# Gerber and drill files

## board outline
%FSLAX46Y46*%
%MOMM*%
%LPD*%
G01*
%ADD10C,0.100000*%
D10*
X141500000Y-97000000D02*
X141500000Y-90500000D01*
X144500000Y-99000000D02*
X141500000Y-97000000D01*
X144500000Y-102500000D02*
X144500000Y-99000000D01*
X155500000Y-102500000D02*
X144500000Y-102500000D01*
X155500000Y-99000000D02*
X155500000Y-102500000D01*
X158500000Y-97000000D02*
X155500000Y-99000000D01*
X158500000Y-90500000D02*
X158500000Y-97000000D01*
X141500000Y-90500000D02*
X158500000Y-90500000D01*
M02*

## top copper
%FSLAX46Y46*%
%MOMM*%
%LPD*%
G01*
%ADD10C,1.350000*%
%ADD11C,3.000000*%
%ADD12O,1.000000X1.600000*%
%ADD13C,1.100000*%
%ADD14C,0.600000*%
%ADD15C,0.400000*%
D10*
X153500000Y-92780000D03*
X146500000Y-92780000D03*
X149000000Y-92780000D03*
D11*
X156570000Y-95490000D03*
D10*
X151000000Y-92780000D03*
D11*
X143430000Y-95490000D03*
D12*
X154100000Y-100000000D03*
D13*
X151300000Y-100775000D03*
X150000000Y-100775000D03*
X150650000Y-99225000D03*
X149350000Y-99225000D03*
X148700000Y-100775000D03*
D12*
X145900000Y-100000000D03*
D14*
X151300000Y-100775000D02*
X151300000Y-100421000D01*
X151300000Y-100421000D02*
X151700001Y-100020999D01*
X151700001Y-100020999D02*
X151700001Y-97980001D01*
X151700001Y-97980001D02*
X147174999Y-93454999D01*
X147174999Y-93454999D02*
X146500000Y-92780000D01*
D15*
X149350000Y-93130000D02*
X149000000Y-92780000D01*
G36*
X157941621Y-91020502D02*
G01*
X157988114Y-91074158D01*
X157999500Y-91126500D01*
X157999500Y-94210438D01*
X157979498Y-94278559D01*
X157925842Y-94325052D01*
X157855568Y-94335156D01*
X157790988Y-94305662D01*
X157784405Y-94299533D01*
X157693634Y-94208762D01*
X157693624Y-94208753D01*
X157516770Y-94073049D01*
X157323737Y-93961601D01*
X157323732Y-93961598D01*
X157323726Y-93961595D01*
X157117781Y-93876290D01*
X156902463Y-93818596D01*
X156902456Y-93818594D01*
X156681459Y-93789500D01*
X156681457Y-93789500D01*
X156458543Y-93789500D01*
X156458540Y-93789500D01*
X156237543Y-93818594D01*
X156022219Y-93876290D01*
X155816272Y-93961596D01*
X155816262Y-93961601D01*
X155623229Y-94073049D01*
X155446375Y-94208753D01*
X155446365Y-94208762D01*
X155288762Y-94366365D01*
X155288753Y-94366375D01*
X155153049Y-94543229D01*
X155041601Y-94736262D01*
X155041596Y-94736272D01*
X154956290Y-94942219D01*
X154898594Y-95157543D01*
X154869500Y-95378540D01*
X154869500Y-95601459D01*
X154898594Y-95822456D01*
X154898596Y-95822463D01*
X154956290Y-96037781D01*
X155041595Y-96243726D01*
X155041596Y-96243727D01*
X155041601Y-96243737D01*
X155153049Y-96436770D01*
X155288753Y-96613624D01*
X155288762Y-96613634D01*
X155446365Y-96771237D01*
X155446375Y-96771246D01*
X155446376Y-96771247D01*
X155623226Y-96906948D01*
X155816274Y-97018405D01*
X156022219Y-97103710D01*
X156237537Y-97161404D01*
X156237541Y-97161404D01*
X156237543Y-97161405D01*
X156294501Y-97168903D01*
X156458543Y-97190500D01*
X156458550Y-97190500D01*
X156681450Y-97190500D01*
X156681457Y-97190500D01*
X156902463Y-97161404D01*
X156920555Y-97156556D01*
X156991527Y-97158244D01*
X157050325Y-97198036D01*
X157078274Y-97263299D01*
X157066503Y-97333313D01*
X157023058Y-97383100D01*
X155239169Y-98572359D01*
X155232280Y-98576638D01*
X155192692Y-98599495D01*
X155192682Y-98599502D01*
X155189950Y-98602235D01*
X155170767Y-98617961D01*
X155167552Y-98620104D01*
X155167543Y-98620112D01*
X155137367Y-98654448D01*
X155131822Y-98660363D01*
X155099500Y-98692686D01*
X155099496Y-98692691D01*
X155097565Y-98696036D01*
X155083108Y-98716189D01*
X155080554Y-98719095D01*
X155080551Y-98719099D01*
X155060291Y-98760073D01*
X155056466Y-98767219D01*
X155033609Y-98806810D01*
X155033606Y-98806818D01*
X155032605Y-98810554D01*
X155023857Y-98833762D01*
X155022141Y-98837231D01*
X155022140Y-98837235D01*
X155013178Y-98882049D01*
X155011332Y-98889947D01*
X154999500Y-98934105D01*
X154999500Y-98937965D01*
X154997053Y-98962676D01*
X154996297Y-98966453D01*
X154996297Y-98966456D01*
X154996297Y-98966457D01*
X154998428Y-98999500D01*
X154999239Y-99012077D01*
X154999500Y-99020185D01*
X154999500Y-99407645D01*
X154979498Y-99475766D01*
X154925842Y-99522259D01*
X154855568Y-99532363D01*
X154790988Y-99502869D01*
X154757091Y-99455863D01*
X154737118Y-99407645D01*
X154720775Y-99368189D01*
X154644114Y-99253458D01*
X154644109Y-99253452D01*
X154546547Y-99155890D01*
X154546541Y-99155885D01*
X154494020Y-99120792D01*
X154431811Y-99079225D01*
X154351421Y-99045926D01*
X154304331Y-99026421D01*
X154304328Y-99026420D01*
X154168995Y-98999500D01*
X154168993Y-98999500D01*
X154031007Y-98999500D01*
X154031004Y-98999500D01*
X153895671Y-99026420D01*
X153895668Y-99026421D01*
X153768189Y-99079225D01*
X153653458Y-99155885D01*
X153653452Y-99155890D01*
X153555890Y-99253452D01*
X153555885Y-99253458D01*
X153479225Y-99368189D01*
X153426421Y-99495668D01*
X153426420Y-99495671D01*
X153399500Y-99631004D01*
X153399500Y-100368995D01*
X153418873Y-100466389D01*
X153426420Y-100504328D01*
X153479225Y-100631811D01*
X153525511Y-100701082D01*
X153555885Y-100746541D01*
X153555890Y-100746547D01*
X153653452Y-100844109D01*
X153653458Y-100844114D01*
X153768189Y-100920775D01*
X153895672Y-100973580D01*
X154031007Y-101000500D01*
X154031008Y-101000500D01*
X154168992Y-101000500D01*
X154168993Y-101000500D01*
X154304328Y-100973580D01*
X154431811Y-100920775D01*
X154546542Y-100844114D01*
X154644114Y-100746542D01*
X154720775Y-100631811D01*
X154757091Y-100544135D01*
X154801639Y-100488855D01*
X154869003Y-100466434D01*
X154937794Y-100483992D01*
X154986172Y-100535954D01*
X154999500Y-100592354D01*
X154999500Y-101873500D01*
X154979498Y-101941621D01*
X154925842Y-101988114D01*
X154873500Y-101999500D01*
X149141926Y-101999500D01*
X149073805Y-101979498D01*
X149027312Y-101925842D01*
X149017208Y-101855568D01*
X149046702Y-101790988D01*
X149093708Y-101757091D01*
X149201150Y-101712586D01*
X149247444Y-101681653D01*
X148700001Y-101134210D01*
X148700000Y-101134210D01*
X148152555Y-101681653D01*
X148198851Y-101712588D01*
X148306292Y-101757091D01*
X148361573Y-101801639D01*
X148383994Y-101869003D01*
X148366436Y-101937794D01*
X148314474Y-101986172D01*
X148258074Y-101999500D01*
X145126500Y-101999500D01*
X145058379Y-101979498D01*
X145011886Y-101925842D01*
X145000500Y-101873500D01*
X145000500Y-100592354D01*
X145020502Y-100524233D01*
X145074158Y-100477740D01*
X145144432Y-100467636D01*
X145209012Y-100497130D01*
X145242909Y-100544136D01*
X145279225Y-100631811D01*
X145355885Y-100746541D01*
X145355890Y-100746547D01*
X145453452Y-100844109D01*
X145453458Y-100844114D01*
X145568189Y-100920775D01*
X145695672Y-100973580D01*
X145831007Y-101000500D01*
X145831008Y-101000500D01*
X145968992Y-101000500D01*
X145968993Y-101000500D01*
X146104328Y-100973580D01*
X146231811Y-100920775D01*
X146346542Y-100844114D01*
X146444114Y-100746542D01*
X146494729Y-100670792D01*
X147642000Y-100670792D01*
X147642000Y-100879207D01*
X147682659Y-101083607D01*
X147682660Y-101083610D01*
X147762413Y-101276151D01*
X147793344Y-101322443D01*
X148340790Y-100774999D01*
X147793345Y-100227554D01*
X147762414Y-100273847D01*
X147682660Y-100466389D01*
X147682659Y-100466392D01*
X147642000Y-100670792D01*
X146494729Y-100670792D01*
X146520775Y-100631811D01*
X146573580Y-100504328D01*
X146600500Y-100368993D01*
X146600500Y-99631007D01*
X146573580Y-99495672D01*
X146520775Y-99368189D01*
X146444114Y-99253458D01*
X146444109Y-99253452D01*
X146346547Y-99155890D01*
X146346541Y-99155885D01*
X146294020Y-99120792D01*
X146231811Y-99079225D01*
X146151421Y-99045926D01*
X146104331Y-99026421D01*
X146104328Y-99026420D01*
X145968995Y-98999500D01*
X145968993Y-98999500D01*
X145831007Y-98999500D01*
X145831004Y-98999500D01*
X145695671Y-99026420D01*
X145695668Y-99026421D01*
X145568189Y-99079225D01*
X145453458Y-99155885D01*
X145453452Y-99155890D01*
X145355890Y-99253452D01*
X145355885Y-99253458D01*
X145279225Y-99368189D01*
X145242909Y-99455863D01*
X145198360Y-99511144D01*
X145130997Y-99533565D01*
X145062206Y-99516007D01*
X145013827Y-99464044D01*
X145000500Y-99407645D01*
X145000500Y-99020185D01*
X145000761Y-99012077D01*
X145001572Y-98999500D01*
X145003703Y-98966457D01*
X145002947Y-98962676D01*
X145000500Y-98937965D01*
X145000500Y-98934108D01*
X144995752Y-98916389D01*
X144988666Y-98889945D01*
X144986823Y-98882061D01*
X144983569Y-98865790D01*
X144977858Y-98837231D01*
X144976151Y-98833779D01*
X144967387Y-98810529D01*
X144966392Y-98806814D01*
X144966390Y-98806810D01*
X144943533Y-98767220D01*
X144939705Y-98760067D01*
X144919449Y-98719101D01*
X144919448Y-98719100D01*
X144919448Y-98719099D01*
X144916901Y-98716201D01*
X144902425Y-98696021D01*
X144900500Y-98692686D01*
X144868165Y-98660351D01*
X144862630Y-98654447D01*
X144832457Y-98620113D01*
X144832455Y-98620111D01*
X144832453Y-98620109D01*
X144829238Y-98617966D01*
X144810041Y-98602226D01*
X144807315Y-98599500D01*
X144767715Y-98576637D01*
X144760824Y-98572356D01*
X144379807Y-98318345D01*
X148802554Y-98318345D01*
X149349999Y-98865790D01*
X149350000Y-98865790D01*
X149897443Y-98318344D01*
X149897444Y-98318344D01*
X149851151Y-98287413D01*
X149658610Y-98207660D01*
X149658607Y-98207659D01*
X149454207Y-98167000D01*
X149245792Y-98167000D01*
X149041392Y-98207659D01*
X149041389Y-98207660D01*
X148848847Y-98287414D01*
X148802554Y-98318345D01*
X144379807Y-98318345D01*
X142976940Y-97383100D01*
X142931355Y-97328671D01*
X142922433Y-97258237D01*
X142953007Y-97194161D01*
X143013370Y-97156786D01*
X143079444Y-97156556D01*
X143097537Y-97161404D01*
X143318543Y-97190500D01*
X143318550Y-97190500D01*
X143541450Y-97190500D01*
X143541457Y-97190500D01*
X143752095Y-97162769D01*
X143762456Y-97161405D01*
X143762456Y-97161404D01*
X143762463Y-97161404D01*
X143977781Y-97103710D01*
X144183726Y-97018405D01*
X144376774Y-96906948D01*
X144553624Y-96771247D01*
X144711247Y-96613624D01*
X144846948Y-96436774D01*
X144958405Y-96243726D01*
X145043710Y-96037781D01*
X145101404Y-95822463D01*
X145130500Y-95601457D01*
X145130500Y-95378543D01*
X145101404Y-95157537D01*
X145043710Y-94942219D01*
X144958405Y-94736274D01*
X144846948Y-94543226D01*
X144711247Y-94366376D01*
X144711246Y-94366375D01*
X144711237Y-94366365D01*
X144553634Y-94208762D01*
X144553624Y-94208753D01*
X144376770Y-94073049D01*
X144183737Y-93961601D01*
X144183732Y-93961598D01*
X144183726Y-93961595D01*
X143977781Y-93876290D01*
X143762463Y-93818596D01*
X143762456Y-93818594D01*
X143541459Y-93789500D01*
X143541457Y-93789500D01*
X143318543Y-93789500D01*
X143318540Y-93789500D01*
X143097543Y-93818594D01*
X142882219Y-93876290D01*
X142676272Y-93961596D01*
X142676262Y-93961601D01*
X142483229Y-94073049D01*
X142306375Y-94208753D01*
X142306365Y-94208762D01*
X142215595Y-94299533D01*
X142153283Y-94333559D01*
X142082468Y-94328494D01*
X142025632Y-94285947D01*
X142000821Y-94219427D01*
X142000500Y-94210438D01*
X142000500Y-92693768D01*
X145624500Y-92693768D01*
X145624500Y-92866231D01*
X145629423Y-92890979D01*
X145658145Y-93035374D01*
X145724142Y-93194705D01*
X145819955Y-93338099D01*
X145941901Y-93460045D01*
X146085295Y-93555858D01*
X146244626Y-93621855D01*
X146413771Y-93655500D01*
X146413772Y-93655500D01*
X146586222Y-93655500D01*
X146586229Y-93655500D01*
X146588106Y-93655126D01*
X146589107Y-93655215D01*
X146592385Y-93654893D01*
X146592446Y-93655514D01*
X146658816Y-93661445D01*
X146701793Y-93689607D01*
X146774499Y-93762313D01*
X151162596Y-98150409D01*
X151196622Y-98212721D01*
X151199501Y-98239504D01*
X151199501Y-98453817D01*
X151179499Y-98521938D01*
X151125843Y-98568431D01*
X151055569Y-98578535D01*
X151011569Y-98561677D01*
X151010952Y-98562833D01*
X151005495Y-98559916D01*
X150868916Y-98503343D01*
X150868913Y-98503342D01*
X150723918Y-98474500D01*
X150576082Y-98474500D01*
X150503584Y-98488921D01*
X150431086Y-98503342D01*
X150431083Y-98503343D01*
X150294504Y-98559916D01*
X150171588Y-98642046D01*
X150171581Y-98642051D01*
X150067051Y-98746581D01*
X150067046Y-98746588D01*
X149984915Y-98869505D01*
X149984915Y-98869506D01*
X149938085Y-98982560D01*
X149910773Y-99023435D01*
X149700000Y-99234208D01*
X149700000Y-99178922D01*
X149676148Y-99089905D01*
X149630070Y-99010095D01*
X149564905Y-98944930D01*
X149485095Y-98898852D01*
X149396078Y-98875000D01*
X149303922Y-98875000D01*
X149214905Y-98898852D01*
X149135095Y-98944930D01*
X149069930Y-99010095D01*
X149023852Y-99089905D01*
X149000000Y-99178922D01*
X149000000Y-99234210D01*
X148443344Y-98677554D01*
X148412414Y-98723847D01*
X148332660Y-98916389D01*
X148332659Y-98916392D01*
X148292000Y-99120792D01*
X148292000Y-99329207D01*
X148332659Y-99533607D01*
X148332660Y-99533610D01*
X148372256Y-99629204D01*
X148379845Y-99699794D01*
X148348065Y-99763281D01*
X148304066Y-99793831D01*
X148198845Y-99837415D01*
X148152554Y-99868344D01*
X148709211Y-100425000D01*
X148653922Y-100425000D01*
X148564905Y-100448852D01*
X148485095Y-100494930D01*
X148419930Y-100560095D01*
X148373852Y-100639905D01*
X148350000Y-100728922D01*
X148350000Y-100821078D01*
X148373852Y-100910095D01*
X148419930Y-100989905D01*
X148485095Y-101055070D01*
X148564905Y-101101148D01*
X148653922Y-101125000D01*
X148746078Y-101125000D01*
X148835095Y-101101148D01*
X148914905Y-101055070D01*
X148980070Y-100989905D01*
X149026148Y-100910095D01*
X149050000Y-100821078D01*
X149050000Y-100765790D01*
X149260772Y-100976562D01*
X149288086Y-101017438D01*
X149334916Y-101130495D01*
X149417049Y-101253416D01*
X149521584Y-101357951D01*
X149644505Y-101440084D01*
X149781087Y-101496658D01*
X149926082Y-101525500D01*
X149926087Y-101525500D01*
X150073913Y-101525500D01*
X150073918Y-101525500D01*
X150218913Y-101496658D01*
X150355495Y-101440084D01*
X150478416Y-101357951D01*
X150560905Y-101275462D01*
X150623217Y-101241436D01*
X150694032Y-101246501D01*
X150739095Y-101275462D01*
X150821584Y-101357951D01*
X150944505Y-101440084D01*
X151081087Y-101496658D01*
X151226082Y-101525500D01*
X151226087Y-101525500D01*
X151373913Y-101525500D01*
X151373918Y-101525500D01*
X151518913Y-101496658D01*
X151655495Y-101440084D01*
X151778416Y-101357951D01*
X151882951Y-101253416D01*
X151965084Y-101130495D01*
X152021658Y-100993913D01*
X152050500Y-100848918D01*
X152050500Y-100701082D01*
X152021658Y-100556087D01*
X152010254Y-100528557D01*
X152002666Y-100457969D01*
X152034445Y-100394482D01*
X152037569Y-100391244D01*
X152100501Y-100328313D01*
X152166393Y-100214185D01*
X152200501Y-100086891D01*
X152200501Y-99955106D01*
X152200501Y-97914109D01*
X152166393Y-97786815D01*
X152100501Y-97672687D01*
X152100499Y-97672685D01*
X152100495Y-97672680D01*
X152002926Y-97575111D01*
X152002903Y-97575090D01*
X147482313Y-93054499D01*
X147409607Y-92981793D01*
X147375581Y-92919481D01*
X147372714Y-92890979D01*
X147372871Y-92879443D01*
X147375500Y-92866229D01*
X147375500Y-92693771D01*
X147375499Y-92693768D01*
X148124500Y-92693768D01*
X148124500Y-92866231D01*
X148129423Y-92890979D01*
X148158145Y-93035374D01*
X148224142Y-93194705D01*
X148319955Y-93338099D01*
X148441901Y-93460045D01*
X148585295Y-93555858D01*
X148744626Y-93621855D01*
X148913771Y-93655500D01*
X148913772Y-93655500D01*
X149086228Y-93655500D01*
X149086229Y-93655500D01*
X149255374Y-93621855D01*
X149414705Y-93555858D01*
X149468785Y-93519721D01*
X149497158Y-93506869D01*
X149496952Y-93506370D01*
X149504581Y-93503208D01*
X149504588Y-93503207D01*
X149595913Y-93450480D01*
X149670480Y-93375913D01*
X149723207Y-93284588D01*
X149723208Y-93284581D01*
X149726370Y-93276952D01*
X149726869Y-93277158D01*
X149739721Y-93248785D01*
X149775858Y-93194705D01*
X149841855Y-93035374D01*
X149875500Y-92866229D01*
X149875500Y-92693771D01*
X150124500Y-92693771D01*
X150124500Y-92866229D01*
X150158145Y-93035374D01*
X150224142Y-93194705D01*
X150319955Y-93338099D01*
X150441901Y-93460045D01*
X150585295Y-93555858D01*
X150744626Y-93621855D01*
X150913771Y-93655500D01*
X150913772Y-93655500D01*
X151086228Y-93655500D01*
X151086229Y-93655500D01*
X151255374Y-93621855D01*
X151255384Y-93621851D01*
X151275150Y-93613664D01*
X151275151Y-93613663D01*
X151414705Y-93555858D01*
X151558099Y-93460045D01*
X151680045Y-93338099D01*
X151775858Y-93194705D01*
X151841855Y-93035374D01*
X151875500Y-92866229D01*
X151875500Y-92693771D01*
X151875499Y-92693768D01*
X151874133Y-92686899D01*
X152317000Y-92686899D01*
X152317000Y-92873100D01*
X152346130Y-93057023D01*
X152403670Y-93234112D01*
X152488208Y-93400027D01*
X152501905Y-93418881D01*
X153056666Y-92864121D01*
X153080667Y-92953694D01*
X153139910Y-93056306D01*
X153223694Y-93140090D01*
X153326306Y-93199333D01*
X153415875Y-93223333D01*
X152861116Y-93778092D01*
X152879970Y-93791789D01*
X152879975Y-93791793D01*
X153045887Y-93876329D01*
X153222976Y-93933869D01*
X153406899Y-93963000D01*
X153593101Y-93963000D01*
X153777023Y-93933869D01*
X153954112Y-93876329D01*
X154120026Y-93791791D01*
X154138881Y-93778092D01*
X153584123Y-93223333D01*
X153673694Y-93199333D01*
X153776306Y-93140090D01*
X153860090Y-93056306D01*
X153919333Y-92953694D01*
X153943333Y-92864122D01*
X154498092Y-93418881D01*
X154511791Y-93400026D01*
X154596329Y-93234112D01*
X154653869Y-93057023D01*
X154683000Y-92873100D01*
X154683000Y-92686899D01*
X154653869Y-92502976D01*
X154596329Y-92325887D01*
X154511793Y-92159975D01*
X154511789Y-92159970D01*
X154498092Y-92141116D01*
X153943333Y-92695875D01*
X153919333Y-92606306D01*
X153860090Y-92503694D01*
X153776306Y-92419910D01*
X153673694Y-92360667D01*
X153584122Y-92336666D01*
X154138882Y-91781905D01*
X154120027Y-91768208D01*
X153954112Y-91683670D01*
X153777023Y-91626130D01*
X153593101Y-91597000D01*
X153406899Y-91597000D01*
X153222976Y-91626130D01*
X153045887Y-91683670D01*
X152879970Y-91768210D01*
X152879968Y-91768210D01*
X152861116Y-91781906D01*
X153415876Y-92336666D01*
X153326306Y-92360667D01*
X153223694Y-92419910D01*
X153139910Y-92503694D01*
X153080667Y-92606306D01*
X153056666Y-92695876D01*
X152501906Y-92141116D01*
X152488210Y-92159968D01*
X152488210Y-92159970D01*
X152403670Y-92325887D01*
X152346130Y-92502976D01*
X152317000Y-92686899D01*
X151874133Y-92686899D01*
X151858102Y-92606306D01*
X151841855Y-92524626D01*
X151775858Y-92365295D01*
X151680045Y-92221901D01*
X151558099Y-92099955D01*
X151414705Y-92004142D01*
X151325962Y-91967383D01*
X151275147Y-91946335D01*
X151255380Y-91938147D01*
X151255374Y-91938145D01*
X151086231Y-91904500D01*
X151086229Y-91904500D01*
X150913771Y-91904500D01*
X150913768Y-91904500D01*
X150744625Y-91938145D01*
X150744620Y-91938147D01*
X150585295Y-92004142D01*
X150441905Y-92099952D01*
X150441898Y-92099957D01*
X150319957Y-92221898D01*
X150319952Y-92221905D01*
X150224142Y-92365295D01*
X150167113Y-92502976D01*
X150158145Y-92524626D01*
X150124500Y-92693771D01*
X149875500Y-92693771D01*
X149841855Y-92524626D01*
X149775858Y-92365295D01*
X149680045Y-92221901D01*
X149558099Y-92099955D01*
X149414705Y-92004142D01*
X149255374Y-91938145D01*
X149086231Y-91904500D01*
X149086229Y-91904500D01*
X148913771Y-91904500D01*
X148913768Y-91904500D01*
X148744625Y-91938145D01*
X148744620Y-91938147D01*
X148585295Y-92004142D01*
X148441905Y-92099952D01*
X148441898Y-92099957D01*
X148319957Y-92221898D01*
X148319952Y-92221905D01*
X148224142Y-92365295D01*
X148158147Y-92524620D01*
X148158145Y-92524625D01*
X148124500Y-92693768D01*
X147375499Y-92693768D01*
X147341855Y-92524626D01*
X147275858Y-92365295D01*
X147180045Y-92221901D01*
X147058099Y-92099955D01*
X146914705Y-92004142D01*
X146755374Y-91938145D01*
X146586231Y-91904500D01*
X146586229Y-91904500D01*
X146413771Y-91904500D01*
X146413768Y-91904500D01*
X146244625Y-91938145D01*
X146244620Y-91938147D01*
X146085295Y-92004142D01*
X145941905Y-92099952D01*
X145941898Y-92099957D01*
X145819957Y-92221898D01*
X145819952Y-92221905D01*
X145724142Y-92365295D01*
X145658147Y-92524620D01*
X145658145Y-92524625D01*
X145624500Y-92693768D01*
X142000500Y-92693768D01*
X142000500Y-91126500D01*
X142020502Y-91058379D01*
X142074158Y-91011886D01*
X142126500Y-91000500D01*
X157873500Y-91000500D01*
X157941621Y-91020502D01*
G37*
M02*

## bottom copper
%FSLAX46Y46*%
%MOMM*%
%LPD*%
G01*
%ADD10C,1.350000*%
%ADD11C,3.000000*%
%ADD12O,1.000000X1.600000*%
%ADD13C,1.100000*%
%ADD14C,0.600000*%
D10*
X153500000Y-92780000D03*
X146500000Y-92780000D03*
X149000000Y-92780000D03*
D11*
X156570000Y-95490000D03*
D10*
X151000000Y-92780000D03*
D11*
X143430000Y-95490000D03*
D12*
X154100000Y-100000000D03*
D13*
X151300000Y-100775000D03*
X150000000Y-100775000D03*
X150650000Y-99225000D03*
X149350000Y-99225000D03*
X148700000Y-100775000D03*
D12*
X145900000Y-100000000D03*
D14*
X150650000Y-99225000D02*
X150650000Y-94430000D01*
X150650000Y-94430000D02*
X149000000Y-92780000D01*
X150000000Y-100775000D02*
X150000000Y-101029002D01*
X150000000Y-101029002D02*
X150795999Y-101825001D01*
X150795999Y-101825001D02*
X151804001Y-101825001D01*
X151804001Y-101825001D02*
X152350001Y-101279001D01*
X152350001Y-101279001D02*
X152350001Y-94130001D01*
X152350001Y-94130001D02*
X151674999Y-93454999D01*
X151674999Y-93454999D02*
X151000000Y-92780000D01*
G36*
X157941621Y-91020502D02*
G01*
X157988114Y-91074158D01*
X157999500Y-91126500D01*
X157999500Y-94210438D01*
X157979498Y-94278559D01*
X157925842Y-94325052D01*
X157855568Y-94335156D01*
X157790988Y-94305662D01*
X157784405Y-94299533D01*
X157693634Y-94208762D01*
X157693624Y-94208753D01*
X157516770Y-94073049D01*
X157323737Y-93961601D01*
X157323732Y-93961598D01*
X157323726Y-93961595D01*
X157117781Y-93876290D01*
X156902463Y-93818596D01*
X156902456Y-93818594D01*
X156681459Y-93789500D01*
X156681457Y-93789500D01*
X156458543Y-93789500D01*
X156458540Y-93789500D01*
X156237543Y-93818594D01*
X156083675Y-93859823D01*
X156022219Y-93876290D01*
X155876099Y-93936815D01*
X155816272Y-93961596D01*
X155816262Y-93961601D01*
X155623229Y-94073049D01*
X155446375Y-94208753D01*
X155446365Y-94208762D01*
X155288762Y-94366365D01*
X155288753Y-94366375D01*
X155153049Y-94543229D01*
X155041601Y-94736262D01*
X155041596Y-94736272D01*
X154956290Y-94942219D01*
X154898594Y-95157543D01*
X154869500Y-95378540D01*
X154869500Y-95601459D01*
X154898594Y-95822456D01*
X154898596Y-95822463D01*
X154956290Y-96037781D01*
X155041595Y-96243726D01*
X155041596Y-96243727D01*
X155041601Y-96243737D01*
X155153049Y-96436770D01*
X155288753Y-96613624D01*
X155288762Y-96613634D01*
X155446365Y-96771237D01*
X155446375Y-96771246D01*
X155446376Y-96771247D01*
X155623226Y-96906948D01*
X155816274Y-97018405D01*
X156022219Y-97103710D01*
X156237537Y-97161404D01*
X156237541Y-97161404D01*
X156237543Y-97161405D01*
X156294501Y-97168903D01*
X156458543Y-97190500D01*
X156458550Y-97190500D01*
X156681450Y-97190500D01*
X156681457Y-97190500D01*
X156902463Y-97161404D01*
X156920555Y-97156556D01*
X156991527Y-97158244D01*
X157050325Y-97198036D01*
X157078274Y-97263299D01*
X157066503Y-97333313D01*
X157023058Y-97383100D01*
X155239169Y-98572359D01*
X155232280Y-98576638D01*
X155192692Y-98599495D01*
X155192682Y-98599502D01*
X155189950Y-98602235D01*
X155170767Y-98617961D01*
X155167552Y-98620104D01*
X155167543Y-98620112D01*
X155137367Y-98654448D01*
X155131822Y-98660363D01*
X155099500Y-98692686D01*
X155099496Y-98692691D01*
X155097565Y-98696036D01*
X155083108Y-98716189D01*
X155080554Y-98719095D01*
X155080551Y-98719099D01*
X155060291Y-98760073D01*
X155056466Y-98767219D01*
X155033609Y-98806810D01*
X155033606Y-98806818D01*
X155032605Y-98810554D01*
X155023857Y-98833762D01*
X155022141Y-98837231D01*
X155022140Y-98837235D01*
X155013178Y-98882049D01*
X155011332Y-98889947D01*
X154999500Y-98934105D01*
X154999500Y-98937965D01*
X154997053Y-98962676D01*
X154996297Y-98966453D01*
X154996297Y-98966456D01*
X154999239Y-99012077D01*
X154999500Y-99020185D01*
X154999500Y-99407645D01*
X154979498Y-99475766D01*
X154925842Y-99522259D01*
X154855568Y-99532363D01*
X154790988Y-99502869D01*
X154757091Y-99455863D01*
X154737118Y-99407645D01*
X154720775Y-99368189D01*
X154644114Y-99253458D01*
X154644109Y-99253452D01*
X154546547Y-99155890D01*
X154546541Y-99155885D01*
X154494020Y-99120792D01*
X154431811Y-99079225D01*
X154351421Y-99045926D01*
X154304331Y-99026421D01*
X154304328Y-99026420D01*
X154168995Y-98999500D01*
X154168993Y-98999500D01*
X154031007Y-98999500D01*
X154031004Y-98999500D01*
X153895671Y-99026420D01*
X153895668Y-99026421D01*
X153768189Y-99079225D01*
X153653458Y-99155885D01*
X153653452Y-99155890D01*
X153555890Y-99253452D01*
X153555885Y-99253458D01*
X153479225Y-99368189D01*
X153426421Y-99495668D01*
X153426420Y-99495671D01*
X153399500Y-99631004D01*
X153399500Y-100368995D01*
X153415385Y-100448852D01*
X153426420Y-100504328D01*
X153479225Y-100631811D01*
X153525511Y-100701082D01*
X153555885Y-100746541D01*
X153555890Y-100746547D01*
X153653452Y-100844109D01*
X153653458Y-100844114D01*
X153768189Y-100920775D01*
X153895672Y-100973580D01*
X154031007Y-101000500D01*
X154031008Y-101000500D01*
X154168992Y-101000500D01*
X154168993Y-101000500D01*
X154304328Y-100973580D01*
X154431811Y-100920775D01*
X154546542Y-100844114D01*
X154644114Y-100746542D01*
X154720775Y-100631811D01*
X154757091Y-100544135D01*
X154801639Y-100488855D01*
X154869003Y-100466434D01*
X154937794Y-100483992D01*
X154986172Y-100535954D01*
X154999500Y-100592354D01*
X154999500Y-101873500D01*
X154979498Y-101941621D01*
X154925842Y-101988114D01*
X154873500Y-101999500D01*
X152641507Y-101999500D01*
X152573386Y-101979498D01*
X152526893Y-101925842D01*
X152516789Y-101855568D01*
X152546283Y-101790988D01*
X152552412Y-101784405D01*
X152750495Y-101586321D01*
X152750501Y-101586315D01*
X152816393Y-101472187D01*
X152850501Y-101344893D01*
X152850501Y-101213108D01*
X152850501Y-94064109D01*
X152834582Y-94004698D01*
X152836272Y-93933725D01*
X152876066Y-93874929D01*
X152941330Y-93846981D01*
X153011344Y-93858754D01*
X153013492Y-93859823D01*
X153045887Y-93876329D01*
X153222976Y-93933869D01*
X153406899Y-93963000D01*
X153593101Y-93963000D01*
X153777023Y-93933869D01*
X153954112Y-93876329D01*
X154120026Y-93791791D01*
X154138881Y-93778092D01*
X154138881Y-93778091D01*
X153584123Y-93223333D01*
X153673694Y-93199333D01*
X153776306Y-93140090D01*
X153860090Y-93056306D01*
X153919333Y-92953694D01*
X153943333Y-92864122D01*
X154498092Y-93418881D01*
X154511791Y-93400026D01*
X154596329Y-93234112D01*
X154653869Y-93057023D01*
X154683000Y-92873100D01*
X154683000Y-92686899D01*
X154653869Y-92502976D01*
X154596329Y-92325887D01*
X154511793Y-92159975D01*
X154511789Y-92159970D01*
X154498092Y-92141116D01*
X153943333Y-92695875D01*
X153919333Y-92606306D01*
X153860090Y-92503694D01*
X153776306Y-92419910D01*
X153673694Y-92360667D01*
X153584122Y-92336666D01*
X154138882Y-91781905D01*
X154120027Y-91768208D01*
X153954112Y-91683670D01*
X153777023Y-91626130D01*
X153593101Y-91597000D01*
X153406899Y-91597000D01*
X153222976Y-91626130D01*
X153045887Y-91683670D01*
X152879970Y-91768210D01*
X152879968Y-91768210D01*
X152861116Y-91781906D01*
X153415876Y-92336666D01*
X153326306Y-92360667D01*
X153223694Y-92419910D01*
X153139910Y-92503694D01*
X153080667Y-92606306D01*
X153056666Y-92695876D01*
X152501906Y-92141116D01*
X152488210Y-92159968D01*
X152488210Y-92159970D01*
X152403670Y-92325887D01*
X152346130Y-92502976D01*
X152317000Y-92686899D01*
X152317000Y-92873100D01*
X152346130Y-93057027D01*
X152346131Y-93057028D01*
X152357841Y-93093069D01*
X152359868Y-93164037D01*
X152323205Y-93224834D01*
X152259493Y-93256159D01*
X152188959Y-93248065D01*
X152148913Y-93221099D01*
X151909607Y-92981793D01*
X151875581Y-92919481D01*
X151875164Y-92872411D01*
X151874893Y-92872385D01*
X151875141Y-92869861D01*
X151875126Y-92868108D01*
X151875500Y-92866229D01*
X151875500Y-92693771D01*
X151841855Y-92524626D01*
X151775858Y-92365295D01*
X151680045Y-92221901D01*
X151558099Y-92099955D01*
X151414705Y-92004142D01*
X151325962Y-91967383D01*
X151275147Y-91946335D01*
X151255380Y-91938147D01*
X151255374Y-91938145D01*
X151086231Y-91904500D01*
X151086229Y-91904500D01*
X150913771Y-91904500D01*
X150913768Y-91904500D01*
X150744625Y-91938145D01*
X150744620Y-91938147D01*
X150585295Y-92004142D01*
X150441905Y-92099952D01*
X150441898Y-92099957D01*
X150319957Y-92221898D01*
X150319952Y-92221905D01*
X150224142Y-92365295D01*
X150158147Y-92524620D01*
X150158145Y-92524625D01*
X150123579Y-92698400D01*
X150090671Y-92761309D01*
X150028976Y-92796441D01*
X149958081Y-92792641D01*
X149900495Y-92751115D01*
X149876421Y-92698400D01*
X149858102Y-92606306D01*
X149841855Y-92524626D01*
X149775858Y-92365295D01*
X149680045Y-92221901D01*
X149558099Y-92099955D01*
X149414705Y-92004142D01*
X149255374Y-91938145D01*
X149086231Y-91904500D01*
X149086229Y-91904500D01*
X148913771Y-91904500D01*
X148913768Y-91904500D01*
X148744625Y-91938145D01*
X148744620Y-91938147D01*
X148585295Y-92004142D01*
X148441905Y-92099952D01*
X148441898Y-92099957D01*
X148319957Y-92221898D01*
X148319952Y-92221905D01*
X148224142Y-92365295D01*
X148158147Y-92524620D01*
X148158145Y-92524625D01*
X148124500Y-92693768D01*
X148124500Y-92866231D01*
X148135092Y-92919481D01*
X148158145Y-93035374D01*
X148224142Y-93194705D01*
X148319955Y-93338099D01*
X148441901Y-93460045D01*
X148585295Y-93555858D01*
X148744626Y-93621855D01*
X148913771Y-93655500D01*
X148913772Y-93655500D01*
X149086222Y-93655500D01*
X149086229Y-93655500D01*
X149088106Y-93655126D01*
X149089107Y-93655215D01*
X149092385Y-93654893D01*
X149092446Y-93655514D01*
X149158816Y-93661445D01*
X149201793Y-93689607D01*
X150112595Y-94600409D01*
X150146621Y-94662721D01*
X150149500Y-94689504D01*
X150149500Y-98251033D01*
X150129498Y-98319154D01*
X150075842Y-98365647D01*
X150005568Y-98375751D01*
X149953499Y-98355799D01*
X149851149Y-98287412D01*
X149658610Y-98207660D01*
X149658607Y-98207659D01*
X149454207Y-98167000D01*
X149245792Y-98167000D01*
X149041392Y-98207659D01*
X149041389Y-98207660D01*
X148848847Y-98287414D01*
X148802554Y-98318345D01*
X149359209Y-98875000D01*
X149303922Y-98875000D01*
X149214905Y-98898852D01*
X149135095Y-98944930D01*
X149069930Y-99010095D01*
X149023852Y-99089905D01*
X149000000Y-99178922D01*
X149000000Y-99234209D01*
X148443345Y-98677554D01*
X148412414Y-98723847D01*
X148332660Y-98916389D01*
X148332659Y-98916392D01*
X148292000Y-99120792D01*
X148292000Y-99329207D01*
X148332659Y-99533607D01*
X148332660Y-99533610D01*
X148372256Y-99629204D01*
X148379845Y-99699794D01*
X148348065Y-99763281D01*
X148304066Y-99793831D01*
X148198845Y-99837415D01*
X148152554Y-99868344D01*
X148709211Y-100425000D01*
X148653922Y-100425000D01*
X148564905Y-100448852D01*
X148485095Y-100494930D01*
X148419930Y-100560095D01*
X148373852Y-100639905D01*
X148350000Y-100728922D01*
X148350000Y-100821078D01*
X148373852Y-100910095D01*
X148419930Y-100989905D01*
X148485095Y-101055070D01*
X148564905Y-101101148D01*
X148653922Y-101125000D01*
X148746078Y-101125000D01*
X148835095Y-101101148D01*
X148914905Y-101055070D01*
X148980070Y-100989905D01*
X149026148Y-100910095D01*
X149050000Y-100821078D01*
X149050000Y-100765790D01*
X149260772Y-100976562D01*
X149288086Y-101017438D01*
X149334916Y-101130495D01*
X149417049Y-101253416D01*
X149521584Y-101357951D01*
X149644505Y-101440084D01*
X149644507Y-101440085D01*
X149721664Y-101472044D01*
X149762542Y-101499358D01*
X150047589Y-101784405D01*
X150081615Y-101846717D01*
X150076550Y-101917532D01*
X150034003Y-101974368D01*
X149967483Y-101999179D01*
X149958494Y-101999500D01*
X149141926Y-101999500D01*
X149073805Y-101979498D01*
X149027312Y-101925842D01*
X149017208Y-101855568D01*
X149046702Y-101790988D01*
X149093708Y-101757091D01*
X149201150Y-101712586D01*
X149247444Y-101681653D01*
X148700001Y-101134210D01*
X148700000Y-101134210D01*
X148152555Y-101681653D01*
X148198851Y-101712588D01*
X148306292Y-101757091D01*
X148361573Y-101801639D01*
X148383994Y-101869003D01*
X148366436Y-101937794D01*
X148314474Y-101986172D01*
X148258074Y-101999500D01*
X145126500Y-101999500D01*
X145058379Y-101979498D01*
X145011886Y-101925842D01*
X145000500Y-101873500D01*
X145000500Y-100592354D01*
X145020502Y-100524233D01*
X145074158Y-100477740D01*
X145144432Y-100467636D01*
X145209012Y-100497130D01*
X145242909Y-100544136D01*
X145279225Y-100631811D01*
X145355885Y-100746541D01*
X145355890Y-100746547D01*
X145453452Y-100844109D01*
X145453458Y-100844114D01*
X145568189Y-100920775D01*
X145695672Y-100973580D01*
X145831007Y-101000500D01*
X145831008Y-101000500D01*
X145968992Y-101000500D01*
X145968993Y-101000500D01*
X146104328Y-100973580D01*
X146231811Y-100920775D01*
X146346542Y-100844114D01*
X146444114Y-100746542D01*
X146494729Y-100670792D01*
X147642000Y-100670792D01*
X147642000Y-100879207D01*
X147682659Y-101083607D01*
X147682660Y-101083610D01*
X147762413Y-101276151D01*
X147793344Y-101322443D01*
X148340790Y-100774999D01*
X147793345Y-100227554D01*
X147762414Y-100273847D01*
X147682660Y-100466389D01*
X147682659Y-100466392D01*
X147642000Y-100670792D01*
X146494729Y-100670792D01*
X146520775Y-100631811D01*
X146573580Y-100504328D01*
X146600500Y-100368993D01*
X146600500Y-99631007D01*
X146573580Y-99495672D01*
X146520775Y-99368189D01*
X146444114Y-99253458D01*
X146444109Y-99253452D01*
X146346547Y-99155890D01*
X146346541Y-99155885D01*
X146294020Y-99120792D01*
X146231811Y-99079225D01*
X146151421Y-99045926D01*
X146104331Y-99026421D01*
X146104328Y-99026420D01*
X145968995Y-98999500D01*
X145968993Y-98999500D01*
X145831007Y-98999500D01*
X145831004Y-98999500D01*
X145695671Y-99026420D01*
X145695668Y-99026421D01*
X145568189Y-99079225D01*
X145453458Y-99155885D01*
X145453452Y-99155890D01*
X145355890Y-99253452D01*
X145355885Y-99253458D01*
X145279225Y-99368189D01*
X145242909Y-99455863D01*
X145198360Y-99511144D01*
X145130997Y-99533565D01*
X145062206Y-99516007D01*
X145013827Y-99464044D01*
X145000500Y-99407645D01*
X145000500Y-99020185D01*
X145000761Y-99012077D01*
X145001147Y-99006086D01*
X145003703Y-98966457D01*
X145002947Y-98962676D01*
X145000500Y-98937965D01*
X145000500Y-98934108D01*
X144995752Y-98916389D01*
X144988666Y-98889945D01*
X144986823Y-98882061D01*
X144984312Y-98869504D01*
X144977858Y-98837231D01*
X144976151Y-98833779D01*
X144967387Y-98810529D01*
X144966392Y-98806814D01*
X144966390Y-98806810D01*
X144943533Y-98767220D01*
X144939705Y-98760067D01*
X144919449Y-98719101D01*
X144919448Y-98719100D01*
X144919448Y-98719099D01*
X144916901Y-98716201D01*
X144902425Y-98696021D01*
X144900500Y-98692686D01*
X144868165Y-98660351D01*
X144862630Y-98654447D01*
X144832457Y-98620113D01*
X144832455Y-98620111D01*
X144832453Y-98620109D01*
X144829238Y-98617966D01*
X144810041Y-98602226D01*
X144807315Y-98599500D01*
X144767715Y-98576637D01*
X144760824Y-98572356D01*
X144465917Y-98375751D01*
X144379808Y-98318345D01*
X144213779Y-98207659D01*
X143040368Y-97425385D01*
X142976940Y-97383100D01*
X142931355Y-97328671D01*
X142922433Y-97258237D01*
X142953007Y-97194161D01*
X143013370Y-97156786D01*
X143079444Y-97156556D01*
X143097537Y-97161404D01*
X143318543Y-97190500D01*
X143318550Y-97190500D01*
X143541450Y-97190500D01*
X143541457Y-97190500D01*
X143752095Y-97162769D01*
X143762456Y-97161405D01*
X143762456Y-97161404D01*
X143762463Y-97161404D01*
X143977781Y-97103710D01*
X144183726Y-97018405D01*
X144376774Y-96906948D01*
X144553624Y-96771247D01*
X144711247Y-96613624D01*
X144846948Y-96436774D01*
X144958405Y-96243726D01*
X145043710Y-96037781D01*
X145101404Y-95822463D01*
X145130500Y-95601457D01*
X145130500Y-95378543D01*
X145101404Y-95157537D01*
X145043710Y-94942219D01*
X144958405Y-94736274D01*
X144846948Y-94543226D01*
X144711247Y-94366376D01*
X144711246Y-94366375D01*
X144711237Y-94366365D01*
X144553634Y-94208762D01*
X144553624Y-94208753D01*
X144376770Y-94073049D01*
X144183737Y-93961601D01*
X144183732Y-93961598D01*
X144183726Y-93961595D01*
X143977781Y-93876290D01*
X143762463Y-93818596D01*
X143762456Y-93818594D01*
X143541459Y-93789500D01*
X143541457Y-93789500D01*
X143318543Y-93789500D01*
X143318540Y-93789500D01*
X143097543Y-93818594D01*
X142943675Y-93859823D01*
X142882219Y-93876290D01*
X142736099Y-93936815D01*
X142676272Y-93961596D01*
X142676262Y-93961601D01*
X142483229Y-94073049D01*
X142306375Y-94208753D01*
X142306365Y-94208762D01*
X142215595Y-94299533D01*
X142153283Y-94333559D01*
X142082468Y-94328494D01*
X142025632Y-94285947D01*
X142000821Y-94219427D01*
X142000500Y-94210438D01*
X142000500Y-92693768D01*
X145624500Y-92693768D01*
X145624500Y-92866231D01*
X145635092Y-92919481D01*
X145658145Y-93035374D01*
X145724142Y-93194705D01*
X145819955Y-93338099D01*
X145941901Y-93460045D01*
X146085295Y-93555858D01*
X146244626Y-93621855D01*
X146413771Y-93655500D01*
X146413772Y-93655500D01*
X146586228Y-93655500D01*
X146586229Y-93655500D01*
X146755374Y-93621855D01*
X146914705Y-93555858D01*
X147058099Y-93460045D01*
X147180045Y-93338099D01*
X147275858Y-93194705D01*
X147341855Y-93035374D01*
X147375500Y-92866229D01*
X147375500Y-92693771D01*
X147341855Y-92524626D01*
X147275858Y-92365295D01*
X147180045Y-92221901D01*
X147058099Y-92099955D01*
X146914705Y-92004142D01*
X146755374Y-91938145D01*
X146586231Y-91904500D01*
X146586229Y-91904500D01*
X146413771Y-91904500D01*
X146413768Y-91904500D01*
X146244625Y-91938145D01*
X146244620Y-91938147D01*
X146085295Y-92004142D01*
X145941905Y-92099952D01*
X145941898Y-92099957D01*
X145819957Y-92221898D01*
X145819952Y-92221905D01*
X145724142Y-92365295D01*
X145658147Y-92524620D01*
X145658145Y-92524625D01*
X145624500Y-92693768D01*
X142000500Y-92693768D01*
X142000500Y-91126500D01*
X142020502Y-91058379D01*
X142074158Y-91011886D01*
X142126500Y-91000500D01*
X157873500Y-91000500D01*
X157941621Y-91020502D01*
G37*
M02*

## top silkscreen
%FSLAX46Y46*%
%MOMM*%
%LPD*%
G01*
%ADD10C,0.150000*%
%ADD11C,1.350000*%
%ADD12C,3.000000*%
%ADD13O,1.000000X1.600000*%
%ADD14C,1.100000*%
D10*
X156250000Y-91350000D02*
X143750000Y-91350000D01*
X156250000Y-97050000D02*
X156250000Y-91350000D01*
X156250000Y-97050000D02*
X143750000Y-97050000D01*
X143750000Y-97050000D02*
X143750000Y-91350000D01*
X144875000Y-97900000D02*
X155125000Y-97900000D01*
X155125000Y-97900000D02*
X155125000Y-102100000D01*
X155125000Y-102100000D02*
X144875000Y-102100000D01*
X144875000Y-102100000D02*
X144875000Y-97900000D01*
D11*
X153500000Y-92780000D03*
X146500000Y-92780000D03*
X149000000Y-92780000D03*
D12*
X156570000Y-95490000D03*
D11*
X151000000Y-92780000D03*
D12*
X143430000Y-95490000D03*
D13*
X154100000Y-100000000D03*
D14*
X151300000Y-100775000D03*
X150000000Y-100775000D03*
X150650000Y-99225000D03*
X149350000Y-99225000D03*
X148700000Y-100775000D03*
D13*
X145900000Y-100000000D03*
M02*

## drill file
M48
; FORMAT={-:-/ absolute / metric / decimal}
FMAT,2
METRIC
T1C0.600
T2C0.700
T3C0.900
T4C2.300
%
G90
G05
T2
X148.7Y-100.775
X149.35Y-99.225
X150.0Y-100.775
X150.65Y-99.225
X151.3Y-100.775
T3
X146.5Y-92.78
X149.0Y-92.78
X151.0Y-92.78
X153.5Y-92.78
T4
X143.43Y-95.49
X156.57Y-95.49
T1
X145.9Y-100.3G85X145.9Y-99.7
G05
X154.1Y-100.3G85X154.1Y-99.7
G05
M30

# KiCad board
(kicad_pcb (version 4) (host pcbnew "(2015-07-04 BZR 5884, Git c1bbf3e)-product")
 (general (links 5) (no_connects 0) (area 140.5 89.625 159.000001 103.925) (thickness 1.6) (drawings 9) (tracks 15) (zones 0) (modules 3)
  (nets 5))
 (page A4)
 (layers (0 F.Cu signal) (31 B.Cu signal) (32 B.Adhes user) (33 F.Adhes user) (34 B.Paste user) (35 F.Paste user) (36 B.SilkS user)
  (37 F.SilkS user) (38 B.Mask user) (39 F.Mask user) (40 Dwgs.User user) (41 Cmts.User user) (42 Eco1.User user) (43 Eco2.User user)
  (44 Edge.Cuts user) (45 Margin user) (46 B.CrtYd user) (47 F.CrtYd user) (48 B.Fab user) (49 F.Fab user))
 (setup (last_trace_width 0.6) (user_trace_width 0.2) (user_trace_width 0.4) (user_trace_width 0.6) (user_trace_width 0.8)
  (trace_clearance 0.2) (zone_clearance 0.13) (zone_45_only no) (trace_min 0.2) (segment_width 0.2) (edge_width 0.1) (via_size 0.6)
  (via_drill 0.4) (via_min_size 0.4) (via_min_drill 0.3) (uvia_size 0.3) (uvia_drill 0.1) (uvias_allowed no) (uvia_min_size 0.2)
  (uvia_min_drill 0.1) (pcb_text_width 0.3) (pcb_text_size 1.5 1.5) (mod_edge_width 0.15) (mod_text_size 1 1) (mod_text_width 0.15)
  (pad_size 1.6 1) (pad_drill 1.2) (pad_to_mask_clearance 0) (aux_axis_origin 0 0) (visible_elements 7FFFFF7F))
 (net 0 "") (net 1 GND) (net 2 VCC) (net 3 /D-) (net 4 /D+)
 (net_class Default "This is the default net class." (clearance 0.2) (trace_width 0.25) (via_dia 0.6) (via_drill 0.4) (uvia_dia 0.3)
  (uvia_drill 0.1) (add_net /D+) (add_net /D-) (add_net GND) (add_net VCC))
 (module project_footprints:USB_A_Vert (layer F.Cu) (at 150 97)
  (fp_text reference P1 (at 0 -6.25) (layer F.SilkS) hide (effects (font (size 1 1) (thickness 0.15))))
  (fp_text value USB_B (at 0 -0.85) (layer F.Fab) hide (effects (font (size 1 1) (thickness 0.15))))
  (fp_line (start 6.25 -5.65) (end -6.25 -5.65) (layer F.SilkS) (width 0.15))
  (fp_line (start 6.25 0.05) (end 6.25 -5.65) (layer F.SilkS) (width 0.15))
  (fp_line (start 6.25 0.05) (end -6.25 0.05) (layer F.SilkS) (width 0.15))
  (fp_line (start -6.25 0.05) (end -6.25 -5.65) (layer F.SilkS) (width 0.15))
  (pad 4 thru_hole circle (at 3.5 -4.22 90) (size 1.35 1.35) (drill 0.9) (layers *.Cu *.Mask F.SilkS) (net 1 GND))
  (pad 1 thru_hole circle (at -3.5 -4.22 90) (size 1.35 1.35) (drill 0.9) (layers *.Cu *.Mask F.SilkS) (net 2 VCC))
  (pad 2 thru_hole circle (at -1 -4.22 90) (size 1.35 1.35) (drill 0.9) (layers *.Cu *.Mask F.SilkS) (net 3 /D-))
  (pad 6 thru_hole circle (at 6.57 -1.51 90) (size 3 3) (drill 2.3) (layers *.Cu *.Mask F.SilkS))
  (pad 3 thru_hole circle (at 1 -4.22 90) (size 1.35 1.35) (drill 0.9) (layers *.Cu *.Mask F.SilkS) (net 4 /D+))
  (pad 6 thru_hole circle (at -6.57 -1.51 90) (size 3 3) (drill 2.3) (layers *.Cu *.Mask F.SilkS)))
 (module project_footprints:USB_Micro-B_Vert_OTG (layer F.Cu) (at 150 100)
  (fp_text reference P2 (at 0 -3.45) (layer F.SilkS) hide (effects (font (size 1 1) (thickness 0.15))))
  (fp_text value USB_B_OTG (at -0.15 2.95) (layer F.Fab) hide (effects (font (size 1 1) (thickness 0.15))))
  (fp_line (start -5.125 -2.1) (end 5.125 -2.1) (layer F.SilkS) (width 0.15))
  (fp_line (start 5.125 -2.1) (end 5.125 2.1) (layer F.SilkS) (width 0.15))
  (fp_line (start 5.125 2.1) (end -5.125 2.1) (layer F.SilkS) (width 0.15))
  (fp_line (start -5.125 2.1) (end -5.125 -2.1) (layer F.SilkS) (width 0.15))
  (pad 6 thru_hole oval (at 4.1 0 90) (size 1.6 1) (drill oval 1.2 0.6) (layers *.Cu *.Mask F.SilkS))
  (pad 1 thru_hole circle (at 1.3 0.775 90) (size 1.1 1.1) (drill 0.7) (layers *.Cu *.Mask F.SilkS) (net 2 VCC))
  (pad 3 thru_hole circle (at 0 0.775 90) (size 1.1 1.1) (drill 0.7) (layers *.Cu *.Mask F.SilkS) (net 4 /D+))
  (pad 2 thru_hole circle (at 0.65 -0.775 90) (size 1.1 1.1) (drill 0.7) (layers *.Cu *.Mask F.SilkS) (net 3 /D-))
  (pad 4 thru_hole circle (at -0.65 -0.775 90) (size 1.1 1.1) (drill 0.7) (layers *.Cu *.Mask F.SilkS) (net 1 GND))
  (pad 5 thru_hole circle (at -1.3 0.775 90) (size 1.1 1.1) (drill 0.7) (layers *.Cu *.Mask F.SilkS) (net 1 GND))
  (pad 6 thru_hole oval (at -4.1 0 90) (size 1.6 1) (drill oval 1.2 0.6) (layers *.Cu *.Mask F.SilkS)))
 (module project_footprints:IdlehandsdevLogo (layer B.Cu) (at 150 96)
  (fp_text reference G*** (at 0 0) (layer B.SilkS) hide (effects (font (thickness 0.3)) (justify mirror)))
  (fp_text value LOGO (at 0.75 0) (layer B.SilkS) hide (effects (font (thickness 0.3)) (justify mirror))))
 (gr_line (start 141.5 97) (end 141.5 90.5) (layer Edge.Cuts) (width 0.1))
 (gr_line (start 144.5 99) (end 141.5 97) (layer Edge.Cuts) (width 0.1))
 (gr_line (start 144.5 102.5) (end 144.5 99) (layer Edge.Cuts) (width 0.1))
 (gr_line (start 155.5 102.5) (end 144.5 102.5) (layer Edge.Cuts) (width 0.1))
 (gr_line (start 155.5 99) (end 155.5 102.5) (layer Edge.Cuts) (width 0.1))
 (gr_line (start 158.5 97) (end 155.5 99) (layer Edge.Cuts) (width 0.1))
 (gr_line (start 158.5 90.5) (end 158.5 97) (layer Edge.Cuts) (width 0.1))
 (gr_line (start 141.5 90.5) (end 158.5 90.5) (layer Edge.Cuts) (width 0.1))
 (segment (start 151.3 100.775) (end 151.3 100.421) (width 0.6) (layer F.Cu) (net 2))
 (segment (start 151.3 100.421) (end 151.700001 100.020999) (width 0.6) (layer F.Cu) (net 2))
 (segment (start 151.700001 100.020999) (end 151.700001 97.980001) (width 0.6) (layer F.Cu) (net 2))
 (segment (start 151.700001 97.980001) (end 147.174999 93.454999) (width 0.6) (layer F.Cu) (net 2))
 (segment (start 147.174999 93.454999) (end 146.5 92.78) (width 0.6) (layer F.Cu) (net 2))
 (segment (start 150.65 99.225) (end 150.65 94.43) (width 0.6) (layer B.Cu) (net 3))
 (segment (start 150.65 94.43) (end 149 92.78) (width 0.6) (layer B.Cu) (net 3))
 (segment (start 149.35 93.13) (end 149 92.78) (width 0.4) (layer F.Cu) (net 3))
 (segment (start 150 100.775) (end 150 101.029002) (width 0.6) (layer B.Cu) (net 4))
 (segment (start 150 101.029002) (end 150.795999 101.825001) (width 0.6) (layer B.Cu) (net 4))
 (segment (start 150.795999 101.825001) (end 151.804001 101.825001) (width 0.6) (layer B.Cu) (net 4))
 (segment (start 151.804001 101.825001) (end 152.350001 101.279001) (width 0.6) (layer B.Cu) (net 4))
 (segment (start 152.350001 101.279001) (end 152.350001 94.130001) (width 0.6) (layer B.Cu) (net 4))
 (segment (start 152.350001 94.130001) (end 151.674999 93.454999) (width 0.6) (layer B.Cu) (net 4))
 (segment (start 151.674999 93.454999) (end 151 92.78) (width 0.6) (layer B.Cu) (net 4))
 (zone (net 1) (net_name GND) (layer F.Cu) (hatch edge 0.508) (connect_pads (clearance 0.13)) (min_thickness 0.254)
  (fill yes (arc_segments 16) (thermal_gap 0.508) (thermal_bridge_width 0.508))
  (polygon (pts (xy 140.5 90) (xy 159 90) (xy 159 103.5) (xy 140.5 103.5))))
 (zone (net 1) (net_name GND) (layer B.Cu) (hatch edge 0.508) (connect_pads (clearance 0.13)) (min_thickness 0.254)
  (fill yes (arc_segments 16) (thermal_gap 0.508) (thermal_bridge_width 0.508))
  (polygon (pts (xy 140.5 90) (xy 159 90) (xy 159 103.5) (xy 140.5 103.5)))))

